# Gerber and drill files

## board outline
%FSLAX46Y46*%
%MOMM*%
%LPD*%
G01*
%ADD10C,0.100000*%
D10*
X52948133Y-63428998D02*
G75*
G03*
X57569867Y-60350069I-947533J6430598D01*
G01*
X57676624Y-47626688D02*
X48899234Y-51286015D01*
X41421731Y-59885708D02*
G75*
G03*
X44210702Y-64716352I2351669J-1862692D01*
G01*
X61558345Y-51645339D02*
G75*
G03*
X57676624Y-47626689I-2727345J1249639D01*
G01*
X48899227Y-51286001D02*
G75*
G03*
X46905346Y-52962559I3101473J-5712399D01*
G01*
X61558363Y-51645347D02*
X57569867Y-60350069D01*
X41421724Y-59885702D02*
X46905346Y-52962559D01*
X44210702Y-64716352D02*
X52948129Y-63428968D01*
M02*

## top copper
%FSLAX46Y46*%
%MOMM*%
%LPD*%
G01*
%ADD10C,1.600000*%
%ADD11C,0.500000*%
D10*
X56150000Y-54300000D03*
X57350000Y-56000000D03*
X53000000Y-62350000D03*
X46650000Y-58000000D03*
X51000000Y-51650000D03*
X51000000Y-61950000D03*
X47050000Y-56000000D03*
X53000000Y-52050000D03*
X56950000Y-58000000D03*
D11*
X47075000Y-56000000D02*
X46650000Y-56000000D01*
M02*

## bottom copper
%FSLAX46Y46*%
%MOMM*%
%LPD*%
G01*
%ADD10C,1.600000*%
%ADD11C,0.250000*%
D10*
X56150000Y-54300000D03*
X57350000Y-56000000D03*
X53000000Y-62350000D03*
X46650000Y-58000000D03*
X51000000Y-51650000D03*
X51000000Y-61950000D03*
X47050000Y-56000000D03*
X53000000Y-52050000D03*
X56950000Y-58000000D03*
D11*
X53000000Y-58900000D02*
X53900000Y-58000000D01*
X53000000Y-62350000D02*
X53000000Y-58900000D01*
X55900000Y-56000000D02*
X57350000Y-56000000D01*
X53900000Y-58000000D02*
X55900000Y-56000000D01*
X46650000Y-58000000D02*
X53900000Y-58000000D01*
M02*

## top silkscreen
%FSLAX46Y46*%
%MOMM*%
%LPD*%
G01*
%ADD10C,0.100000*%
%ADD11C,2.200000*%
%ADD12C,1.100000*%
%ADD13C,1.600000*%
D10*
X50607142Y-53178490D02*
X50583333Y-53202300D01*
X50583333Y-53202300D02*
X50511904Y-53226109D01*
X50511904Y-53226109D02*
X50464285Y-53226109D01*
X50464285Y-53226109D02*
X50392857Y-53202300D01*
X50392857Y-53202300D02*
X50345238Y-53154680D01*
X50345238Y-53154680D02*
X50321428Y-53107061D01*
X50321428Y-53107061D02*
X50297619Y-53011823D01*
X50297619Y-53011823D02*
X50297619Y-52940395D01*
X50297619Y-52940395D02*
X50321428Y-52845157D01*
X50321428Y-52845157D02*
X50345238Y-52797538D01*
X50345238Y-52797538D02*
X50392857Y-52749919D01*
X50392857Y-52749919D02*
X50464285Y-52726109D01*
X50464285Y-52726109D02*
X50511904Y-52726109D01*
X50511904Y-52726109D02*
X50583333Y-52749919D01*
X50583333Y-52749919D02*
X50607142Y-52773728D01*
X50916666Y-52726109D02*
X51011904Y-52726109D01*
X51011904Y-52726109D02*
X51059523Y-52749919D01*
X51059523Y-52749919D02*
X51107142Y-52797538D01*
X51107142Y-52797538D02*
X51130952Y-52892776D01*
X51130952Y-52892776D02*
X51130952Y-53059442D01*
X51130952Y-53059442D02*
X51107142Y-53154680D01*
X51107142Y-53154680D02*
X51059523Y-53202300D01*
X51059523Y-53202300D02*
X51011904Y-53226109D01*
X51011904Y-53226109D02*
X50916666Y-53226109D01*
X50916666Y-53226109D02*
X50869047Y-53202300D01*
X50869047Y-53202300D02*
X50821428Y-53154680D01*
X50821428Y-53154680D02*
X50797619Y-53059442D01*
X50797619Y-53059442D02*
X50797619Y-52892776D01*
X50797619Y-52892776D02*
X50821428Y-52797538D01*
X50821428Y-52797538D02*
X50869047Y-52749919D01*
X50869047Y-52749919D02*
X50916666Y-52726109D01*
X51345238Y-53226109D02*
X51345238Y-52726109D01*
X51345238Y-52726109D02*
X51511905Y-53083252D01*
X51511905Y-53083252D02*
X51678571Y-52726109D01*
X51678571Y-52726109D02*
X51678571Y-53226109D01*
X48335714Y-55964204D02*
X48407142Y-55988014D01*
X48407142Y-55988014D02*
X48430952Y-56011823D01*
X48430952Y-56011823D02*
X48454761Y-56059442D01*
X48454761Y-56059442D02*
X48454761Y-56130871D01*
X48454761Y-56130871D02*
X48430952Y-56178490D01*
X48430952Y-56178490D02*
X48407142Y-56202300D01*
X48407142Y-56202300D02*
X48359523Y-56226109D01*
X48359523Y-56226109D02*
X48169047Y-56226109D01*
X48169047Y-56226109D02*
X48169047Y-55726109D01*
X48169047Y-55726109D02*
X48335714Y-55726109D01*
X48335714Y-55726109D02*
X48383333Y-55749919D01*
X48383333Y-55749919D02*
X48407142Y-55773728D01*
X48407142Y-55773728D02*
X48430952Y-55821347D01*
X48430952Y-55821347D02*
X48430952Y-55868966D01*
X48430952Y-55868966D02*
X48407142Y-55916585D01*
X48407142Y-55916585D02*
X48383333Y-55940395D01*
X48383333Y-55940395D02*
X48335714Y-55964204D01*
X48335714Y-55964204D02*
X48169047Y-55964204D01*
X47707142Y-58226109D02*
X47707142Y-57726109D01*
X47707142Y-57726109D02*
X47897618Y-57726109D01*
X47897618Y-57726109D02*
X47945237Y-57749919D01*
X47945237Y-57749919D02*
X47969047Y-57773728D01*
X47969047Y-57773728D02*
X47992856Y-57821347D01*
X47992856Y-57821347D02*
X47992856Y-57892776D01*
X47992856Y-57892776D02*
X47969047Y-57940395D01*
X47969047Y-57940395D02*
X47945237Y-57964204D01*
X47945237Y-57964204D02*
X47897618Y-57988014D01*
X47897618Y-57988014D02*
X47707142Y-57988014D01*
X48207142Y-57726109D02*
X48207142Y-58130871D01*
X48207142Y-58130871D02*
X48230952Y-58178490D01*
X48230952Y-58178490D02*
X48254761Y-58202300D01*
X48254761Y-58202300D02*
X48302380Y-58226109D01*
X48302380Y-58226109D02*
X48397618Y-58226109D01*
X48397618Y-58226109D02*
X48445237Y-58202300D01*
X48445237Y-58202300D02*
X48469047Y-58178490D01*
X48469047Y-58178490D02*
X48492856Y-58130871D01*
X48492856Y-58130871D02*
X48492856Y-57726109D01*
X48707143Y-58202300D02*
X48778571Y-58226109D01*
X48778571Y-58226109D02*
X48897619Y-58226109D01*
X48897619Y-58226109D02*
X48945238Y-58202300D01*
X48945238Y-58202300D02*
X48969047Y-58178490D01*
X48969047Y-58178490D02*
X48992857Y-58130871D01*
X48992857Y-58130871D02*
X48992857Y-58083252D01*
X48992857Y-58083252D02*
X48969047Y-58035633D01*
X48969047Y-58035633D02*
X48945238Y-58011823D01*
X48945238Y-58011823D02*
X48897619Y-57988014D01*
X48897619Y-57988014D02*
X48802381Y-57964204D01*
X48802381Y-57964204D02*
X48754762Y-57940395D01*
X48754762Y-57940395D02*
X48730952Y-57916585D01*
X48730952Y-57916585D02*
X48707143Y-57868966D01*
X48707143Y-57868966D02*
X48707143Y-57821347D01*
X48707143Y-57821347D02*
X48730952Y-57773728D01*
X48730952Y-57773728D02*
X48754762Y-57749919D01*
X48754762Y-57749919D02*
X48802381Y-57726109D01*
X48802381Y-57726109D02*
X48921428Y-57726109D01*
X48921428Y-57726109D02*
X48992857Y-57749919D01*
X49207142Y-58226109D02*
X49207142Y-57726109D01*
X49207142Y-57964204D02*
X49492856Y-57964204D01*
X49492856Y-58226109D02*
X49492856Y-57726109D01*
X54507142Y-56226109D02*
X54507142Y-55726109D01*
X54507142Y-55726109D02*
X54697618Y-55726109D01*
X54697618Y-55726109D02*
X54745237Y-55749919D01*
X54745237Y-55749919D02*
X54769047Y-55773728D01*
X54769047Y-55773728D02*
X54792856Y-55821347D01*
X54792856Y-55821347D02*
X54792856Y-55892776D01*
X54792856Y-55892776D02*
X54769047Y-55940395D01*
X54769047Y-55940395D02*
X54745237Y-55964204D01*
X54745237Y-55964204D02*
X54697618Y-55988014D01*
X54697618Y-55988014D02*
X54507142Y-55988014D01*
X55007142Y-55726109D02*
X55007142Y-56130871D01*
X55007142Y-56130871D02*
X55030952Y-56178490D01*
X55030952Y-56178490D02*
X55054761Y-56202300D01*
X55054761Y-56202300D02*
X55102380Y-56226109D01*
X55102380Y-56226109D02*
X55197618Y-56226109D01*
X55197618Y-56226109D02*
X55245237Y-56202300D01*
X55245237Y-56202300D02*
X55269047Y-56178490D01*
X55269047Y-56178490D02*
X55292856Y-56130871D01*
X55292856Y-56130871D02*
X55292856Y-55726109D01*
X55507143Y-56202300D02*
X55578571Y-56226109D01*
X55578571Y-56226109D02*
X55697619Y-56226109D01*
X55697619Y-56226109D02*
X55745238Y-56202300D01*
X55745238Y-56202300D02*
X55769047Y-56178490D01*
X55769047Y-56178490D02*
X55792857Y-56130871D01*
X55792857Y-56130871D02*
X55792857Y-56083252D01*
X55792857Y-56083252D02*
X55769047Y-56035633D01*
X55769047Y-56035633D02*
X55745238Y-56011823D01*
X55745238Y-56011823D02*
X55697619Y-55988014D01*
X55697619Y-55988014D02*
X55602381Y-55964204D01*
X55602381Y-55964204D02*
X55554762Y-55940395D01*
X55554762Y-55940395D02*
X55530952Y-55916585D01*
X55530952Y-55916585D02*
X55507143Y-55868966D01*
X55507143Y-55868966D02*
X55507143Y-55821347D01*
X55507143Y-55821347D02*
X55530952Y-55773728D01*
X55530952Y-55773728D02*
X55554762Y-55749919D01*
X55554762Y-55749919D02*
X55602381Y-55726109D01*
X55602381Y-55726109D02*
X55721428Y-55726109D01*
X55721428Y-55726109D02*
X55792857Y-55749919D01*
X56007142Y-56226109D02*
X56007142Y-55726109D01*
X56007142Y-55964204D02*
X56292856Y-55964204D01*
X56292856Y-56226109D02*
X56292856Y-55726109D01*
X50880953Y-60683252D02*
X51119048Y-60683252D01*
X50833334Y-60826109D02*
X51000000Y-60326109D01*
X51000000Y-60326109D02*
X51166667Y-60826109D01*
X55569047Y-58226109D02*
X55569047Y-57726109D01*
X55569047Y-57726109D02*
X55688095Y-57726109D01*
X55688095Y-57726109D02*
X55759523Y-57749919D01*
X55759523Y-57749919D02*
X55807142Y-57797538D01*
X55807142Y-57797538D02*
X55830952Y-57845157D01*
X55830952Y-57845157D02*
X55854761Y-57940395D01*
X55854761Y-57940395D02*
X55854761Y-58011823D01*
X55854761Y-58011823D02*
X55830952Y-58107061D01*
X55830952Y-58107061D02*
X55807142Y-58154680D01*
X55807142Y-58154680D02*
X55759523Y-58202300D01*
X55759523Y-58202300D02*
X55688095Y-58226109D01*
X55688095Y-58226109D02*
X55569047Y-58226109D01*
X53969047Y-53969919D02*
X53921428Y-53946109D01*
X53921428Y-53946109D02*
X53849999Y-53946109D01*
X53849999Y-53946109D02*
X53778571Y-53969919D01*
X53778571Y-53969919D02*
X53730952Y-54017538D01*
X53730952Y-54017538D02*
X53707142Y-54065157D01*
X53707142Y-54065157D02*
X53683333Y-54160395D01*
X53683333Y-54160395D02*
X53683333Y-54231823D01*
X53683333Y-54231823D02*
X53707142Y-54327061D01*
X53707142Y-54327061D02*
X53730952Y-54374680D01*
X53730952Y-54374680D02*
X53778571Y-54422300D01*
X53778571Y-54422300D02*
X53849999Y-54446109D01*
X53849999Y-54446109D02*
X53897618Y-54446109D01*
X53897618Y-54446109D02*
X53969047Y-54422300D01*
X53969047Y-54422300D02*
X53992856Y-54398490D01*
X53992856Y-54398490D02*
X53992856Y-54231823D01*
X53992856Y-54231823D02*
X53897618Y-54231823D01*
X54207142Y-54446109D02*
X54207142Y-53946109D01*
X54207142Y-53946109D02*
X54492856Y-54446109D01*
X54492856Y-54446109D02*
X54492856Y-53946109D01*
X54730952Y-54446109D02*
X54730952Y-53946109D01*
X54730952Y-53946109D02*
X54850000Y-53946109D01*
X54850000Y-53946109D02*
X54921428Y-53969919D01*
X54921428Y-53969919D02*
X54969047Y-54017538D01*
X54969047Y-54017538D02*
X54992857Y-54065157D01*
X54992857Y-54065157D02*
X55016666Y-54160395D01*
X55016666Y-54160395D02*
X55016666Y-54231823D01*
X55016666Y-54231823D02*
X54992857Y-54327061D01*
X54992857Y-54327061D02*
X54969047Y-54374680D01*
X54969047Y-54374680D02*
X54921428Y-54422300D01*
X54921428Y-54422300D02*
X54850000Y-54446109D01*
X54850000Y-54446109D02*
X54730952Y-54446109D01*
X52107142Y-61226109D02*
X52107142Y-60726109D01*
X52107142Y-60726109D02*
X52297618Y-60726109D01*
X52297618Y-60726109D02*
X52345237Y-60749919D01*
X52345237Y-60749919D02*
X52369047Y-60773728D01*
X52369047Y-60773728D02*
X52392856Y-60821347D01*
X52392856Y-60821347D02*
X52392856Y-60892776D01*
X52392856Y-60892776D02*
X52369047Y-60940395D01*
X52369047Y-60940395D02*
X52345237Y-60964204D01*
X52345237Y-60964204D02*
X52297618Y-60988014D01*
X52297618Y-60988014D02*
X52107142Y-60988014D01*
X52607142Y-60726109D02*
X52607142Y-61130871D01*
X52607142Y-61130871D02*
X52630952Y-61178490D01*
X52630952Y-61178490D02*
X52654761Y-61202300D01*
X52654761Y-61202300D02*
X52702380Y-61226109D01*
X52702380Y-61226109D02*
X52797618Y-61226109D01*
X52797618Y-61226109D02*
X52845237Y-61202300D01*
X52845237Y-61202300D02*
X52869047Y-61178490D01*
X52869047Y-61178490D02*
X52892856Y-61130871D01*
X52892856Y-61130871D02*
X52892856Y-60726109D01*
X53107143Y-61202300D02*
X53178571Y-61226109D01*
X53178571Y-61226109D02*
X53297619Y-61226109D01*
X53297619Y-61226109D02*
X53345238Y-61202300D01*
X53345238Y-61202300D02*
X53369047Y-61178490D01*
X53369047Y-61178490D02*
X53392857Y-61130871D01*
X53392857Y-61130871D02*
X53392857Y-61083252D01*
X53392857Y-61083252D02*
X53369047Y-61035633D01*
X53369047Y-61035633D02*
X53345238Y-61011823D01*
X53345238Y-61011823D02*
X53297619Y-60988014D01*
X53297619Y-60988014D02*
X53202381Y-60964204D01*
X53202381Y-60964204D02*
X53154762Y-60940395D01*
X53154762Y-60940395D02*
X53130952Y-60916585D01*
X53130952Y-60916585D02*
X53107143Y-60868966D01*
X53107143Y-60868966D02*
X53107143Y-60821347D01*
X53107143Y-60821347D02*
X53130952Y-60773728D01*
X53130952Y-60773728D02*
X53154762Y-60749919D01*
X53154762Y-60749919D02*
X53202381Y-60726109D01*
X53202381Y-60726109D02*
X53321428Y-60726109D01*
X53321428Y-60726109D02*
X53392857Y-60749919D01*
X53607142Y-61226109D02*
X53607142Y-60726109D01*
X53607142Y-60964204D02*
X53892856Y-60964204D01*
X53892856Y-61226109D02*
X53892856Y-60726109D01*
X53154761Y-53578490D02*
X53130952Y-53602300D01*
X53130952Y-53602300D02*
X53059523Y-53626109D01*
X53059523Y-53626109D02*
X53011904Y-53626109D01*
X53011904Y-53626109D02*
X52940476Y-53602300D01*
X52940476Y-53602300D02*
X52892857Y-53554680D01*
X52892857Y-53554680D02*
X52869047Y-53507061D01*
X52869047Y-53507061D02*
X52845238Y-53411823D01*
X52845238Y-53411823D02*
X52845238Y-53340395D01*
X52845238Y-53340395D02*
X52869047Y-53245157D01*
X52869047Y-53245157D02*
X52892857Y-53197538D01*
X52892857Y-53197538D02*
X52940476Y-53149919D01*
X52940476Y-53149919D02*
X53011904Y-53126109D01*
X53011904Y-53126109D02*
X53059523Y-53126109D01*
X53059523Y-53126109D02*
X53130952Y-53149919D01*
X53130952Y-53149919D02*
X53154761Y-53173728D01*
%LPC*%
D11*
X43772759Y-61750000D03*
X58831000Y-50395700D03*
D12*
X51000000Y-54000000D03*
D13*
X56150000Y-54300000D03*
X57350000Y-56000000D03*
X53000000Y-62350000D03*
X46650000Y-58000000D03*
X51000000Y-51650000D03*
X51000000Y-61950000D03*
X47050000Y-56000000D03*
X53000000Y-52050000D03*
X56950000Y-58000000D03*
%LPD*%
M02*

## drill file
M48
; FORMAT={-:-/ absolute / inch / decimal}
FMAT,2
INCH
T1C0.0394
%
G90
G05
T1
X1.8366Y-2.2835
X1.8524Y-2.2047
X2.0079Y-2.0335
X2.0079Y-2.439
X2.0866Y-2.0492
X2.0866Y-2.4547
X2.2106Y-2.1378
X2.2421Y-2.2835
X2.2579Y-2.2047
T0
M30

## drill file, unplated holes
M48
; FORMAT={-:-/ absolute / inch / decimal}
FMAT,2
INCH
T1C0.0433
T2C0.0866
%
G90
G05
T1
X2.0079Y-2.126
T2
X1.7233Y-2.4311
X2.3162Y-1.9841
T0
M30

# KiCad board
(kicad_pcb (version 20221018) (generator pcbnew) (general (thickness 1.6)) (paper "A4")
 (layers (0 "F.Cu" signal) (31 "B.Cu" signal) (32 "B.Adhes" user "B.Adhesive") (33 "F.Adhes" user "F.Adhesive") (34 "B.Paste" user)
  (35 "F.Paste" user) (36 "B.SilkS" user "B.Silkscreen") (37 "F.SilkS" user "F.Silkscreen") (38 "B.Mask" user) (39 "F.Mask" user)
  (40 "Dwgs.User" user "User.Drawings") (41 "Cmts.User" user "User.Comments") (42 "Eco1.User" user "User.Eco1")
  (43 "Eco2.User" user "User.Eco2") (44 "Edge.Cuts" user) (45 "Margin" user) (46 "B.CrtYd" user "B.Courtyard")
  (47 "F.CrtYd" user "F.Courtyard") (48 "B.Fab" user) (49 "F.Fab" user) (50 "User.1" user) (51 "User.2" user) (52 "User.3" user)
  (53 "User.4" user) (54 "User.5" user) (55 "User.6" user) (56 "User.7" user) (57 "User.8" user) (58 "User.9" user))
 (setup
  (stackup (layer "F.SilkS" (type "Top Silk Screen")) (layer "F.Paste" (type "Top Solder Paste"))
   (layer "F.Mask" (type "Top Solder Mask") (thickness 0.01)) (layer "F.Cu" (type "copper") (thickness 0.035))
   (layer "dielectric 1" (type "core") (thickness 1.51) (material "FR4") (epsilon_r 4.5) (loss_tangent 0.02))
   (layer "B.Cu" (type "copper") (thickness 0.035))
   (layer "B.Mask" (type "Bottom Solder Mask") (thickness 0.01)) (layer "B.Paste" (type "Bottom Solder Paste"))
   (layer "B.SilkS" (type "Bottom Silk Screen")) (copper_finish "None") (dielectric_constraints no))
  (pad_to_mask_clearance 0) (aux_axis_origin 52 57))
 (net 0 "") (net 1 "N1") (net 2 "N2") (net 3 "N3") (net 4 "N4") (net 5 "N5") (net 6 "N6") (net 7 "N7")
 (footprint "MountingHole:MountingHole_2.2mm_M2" (layer "F.Cu") (at 43.772759 61.75)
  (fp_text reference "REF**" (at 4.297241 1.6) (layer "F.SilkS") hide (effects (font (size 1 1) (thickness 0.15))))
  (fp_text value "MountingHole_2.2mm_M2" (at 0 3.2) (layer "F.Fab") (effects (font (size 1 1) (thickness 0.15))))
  (pad "" np_thru_hole circle (at 0 0) (size 2.2 2.2) (drill 2.2) (layers "*.Cu" "*.Mask")))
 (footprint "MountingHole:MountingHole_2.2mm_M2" (layer "F.Cu") (at 58.831 50.3957)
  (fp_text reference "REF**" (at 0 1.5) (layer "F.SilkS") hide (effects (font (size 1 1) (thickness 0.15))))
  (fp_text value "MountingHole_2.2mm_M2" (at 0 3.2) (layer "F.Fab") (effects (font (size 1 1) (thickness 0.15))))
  (pad "" np_thru_hole circle (at 0 0) (size 2.2 2.2) (drill 2.2) (layers "*.Cu" "*.Mask")))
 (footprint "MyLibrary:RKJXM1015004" (layer "B.Cu") (at 52 57 180)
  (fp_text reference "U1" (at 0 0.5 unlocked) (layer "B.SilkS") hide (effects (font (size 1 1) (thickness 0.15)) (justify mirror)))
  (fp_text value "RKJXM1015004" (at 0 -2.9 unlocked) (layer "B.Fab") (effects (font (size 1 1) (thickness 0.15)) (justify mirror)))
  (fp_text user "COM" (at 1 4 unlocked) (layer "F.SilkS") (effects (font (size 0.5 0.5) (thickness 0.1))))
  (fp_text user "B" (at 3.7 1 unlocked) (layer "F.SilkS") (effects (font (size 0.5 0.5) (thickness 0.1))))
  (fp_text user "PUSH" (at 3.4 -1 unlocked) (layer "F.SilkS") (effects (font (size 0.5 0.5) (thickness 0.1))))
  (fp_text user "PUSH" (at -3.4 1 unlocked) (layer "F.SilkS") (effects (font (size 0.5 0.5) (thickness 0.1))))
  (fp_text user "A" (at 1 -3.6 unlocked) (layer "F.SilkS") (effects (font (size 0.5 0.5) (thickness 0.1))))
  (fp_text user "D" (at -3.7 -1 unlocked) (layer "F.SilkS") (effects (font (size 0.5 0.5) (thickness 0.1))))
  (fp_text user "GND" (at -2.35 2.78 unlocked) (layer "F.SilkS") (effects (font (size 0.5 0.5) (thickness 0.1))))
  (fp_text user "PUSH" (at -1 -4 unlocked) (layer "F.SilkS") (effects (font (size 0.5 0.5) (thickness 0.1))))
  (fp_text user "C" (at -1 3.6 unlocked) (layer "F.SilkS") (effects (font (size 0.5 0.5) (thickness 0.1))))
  (pad "" np_thru_hole circle (at 1 3 180) (size 1.1 1.1) (drill 1.1) (layers "F&B.Cu" "*.Mask"))
  (pad "1" thru_hole circle (at -4.15 2.7 180) (size 1.6 1.6) (drill 1) (layers "*.Cu" "*.Mask") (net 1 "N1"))
  (pad "2" thru_hole circle (at -5.35 1 180) (size 1.6 1.6) (drill 1) (layers "*.Cu" "*.Mask") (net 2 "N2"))
  (pad "2" thru_hole circle (at -1 -5.35 180) (size 1.6 1.6) (drill 1) (layers "*.Cu" "*.Mask") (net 2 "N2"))
  (pad "2" thru_hole circle (at 5.35 -1 180) (size 1.6 1.6) (drill 1) (layers "*.Cu" "*.Mask") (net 2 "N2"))
  (pad "3" thru_hole circle (at 1 5.35 180) (size 1.6 1.6) (drill 1) (layers "*.Cu" "*.Mask") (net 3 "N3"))
  (pad "4" thru_hole circle (at 1 -4.95 180) (size 1.6 1.6) (drill 1) (layers "*.Cu" "*.Mask") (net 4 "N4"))
  (pad "5" thru_hole circle (at 4.95 1 180) (size 1.6 1.6) (drill 1) (layers "*.Cu" "*.Mask") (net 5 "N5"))
  (pad "6" thru_hole circle (at -1 4.95 180) (size 1.6 1.6) (drill 1) (layers "*.Cu" "*.Mask") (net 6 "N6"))
  (pad "7" thru_hole circle (at -4.95 -1 180) (size 1.6 1.6) (drill 1) (layers "*.Cu" "*.Mask") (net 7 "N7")))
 (gr_arc (start 57.569867 60.350069) (mid 55.60436 62.407942) (end 52.948129 63.428968) (stroke (width 0.1) (type solid))
  (layer "Edge.Cuts"))
 (gr_line (start 57.676624 47.626688) (end 48.899234 51.286015) (stroke (width 0.1) (type solid)) (layer "Edge.Cuts"))
 (gr_arc (start 44.210702 64.716352) (mid 41.175323 63.248395) (end 41.421724 59.885702) (stroke (width 0.1) (type solid))
  (layer "Edge.Cuts"))
 (gr_arc (start 57.676624 47.626688) (mid 60.988764 48.311458) (end 61.558363 51.645347) (stroke (width 0.1) (type solid))
  (layer "Edge.Cuts"))
 (gr_arc (start 46.905346 52.962559) (mid 47.817439 52.023375) (end 48.899234 51.286015) (stroke (width 0.1) (type solid))
  (layer "Edge.Cuts"))
 (gr_line (start 61.558363 51.645347) (end 57.569867 60.350069) (stroke (width 0.1) (type solid)) (layer "Edge.Cuts"))
 (gr_line (start 41.421724 59.885702) (end 46.905346 52.962559) (stroke (width 0.1) (type solid)) (layer "Edge.Cuts"))
 (gr_line (start 44.210702 64.716352) (end 52.948129 63.428968) (stroke (width 0.1) (type solid)) (layer "Edge.Cuts"))
 (segment (start 53 58.9) (end 53.9 58) (width 0.25) (layer "B.Cu") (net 2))
 (segment (start 53 62.35) (end 53 58.9) (width 0.25) (layer "B.Cu") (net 2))
 (segment (start 55.9 56) (end 57.35 56) (width 0.25) (layer "B.Cu") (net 2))
 (segment (start 53.9 58) (end 55.9 56) (width 0.25) (layer "B.Cu") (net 2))
 (segment (start 46.65 58) (end 53.9 58) (width 0.25) (layer "B.Cu") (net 2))
 (segment (start 47.075 56) (end 46.65 56) (width 0.5) (layer "F.Cu") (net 5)))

